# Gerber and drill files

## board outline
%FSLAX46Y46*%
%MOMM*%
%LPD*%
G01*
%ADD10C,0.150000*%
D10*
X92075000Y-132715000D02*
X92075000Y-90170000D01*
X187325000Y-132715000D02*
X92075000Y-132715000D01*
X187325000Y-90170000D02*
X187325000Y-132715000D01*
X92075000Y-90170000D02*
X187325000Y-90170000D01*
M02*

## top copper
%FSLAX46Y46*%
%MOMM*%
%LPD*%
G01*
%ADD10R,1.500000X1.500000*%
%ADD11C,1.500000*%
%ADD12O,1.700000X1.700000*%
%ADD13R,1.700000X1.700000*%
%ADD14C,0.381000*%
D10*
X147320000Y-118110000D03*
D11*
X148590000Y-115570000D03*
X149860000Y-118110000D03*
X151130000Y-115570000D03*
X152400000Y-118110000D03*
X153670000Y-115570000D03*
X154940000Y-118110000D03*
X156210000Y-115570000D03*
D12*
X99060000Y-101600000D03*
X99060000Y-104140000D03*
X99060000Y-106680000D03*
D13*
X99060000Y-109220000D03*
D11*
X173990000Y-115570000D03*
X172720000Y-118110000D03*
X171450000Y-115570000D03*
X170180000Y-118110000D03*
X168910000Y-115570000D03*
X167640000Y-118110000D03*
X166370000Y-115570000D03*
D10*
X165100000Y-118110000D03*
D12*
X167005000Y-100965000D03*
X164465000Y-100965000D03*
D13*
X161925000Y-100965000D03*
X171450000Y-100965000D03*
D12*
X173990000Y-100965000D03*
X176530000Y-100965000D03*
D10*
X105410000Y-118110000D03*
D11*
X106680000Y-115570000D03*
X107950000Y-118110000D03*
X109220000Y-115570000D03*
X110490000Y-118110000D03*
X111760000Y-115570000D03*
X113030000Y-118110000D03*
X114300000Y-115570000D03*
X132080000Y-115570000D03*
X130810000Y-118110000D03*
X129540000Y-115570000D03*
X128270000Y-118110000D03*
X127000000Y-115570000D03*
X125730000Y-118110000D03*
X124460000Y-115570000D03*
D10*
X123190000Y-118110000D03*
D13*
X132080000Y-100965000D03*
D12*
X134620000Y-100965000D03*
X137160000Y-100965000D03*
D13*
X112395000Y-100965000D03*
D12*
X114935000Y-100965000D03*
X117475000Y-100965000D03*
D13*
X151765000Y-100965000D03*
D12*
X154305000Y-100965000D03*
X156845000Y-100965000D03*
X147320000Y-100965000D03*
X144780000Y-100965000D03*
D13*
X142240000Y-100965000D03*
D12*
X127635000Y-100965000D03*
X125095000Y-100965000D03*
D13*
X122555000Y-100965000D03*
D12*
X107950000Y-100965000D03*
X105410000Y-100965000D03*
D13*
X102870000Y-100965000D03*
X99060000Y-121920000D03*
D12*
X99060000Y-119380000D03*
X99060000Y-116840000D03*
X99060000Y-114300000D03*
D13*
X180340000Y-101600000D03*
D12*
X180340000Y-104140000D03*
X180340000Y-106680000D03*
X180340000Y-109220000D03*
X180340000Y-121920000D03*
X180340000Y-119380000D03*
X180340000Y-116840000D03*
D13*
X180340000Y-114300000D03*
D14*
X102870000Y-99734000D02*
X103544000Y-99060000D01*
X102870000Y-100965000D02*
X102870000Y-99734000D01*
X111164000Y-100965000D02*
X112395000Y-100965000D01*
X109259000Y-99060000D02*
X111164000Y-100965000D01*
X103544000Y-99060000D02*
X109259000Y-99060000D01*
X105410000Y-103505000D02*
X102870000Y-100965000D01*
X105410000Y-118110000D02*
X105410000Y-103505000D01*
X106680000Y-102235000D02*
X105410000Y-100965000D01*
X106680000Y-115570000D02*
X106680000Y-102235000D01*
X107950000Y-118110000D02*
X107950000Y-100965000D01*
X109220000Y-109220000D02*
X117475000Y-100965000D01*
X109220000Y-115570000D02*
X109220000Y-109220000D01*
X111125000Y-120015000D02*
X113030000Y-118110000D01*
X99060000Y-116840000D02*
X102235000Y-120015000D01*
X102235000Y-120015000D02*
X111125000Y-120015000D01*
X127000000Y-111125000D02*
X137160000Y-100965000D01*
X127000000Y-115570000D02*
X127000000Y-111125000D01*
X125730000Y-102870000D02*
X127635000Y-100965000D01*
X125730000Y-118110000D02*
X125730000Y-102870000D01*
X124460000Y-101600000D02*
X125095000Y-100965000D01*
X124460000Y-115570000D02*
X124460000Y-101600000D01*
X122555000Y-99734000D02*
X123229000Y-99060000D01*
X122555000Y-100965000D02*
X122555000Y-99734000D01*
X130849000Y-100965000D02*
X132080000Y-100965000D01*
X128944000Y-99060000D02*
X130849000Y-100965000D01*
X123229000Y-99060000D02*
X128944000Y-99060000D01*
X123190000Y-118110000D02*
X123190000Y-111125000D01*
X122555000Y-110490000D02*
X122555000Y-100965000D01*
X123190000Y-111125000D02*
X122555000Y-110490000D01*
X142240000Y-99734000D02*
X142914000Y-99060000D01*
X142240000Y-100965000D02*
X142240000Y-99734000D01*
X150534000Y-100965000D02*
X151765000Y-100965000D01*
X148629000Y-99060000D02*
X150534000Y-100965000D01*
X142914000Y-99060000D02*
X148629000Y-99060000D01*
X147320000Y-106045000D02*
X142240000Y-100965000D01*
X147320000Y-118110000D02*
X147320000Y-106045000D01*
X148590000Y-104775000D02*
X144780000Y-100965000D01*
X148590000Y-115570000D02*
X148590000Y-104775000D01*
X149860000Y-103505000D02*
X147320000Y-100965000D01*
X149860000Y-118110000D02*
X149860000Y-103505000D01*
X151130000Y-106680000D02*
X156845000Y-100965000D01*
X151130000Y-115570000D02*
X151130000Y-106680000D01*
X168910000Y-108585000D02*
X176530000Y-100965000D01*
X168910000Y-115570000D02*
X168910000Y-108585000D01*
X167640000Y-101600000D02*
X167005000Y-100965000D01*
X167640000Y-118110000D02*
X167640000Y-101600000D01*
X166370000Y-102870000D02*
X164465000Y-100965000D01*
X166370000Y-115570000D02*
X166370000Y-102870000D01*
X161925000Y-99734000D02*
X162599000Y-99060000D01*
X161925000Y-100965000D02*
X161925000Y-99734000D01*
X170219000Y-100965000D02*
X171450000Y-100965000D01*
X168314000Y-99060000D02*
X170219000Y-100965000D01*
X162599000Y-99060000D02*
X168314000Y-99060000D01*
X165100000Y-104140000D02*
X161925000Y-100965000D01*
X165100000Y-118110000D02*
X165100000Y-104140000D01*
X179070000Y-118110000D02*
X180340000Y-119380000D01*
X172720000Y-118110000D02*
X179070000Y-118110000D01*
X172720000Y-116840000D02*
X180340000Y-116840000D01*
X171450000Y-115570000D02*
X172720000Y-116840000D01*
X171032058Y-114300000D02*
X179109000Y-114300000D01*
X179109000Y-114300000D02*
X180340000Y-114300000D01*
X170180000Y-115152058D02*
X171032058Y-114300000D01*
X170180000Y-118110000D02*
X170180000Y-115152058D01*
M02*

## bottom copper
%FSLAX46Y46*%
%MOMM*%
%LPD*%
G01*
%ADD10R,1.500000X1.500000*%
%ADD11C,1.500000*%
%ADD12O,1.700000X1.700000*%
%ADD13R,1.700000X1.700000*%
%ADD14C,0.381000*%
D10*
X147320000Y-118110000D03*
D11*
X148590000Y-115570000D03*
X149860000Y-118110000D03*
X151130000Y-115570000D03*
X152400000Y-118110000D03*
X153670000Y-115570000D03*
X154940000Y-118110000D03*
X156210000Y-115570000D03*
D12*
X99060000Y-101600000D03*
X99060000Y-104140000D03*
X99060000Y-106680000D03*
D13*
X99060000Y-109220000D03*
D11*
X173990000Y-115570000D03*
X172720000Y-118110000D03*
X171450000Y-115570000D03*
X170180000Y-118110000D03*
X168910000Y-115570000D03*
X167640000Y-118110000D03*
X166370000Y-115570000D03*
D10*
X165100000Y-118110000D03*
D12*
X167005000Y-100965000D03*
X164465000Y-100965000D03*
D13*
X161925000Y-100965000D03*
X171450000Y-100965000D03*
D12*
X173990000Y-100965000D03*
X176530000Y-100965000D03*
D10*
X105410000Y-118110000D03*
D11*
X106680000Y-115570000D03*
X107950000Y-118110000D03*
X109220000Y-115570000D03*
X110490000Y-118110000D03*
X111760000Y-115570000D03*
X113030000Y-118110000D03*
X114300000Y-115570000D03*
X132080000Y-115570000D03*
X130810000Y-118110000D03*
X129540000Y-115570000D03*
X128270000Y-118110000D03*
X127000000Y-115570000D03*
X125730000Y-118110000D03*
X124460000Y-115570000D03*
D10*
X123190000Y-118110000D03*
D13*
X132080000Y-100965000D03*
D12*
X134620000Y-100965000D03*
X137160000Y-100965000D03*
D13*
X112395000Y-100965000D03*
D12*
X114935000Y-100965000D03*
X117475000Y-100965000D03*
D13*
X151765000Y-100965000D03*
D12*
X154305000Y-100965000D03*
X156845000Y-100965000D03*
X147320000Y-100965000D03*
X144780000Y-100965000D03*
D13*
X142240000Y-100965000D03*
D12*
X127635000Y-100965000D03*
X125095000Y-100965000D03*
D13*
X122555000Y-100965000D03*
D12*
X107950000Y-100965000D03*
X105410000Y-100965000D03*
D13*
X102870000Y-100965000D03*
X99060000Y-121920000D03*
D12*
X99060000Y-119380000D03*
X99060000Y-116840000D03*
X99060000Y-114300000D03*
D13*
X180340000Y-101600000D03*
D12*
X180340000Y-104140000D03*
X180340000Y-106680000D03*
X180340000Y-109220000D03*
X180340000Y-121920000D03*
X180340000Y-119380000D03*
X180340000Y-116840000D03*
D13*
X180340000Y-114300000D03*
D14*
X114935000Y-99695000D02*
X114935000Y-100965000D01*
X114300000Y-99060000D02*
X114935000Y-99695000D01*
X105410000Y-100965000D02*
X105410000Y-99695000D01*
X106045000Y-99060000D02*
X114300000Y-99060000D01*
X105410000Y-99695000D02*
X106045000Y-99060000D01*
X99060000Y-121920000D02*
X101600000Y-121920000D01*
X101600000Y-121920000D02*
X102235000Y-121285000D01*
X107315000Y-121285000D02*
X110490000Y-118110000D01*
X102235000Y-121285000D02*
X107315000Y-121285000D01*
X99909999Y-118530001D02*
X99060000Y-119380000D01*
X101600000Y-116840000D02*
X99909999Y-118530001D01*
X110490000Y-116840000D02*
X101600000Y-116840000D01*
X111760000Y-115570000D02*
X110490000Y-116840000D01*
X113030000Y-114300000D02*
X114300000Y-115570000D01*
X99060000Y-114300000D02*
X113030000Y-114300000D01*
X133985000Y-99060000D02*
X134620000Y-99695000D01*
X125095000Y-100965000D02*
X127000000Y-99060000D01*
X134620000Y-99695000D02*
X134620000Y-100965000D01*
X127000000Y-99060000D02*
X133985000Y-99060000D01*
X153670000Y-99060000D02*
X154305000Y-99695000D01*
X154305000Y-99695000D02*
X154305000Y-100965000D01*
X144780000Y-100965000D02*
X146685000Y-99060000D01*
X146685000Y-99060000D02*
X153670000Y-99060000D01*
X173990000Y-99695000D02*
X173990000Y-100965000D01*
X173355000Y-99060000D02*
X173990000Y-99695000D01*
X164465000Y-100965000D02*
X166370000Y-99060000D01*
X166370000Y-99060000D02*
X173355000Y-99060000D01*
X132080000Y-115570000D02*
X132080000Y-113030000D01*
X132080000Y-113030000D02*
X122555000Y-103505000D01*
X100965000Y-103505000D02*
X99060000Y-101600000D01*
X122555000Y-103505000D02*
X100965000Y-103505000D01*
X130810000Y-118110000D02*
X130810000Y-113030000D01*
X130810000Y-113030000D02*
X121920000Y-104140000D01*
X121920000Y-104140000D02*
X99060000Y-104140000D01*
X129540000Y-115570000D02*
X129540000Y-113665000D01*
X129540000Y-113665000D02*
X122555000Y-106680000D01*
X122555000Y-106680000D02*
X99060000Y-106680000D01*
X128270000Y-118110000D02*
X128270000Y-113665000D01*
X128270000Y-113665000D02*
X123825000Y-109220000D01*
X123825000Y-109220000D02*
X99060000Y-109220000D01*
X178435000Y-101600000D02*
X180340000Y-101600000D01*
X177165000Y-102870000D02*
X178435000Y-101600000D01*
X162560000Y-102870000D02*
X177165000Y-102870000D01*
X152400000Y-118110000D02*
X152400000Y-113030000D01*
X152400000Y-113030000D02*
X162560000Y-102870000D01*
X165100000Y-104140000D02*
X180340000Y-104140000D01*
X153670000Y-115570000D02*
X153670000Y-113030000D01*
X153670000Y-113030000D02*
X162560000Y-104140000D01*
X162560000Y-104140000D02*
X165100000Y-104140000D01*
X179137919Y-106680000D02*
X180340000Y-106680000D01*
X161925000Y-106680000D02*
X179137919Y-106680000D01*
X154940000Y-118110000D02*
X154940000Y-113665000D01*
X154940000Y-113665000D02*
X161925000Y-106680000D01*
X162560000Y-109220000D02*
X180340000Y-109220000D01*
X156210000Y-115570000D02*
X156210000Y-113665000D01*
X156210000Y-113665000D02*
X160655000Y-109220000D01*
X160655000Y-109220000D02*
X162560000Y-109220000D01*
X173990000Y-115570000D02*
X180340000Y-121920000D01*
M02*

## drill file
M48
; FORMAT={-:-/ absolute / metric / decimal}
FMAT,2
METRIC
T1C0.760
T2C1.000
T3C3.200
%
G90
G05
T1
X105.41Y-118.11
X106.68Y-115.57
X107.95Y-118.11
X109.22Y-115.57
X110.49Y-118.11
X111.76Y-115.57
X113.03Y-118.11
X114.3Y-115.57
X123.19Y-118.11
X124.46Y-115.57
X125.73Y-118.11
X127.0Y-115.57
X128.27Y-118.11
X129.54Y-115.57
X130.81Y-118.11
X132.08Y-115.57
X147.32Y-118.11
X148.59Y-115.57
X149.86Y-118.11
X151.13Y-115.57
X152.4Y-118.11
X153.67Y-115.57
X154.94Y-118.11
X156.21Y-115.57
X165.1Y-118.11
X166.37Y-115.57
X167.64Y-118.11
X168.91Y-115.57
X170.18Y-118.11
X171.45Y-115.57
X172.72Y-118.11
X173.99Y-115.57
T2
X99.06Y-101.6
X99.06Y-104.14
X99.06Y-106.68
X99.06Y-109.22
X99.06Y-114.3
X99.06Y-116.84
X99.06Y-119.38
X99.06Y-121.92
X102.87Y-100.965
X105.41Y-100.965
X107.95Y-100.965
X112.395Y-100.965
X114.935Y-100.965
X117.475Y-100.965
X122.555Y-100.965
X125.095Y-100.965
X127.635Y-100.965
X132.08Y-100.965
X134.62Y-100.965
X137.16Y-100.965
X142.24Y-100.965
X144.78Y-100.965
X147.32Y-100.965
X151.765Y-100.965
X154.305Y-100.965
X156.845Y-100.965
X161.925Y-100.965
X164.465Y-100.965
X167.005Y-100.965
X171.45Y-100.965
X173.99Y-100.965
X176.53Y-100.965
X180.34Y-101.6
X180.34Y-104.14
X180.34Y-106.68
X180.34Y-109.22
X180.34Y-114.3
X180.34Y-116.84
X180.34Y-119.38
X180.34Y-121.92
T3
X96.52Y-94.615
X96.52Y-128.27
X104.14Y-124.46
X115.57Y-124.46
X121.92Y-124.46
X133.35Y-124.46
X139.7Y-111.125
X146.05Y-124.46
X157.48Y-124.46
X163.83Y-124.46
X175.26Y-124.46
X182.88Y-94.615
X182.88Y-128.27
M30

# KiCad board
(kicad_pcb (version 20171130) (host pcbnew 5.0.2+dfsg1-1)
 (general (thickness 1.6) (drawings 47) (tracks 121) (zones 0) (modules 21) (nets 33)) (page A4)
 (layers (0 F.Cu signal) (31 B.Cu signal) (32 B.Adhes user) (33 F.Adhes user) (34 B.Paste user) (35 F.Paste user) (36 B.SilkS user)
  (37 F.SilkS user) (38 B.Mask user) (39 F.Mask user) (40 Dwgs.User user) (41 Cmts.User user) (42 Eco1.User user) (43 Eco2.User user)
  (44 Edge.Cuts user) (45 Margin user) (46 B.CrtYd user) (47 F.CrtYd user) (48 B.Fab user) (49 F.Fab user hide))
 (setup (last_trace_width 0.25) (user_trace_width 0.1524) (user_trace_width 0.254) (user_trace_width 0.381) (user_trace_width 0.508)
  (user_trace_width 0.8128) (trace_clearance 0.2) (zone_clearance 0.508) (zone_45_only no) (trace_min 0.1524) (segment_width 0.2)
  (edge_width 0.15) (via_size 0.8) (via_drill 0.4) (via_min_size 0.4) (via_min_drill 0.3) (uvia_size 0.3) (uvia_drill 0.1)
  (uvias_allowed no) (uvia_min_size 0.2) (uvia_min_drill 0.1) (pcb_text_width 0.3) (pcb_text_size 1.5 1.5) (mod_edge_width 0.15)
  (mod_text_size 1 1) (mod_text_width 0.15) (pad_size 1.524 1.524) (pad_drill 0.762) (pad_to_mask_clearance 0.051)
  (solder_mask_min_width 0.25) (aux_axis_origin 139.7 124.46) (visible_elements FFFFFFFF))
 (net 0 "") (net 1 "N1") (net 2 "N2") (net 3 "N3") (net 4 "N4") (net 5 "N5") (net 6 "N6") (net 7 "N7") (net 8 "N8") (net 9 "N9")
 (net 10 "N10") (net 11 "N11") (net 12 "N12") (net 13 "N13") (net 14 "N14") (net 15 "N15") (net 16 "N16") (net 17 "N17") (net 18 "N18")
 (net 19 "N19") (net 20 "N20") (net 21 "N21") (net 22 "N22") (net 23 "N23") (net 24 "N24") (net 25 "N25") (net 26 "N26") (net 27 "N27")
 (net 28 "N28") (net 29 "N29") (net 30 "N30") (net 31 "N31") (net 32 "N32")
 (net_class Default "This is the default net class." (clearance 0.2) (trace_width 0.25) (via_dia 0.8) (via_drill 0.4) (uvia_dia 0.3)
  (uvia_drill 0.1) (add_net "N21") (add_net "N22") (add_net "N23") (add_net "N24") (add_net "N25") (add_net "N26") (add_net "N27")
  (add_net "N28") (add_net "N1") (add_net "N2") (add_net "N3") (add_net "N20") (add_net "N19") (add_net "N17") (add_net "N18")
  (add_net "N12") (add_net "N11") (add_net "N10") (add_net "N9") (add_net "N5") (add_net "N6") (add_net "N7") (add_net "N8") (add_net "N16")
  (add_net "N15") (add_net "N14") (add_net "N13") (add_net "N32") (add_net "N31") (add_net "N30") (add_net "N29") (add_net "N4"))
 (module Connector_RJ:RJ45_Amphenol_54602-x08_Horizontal (layer F.Cu) (at 147.32 118.11)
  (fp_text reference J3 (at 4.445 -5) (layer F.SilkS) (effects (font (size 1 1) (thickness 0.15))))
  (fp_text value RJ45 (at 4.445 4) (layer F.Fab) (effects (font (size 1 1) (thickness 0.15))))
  (pad "" np_thru_hole circle (at 10.16 6.35) (size 3.2 3.2) (drill 3.2) (layers *.Cu *.Mask))
  (pad "" np_thru_hole circle (at -1.27 6.35) (size 3.2 3.2) (drill 3.2) (layers *.Cu *.Mask))
  (pad 1 thru_hole rect (at 0 0) (size 1.5 1.5) (drill 0.76) (layers *.Cu *.Mask) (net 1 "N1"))
  (pad 2 thru_hole circle (at 1.27 -2.54) (size 1.5 1.5) (drill 0.76) (layers *.Cu *.Mask) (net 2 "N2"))
  (pad 3 thru_hole circle (at 2.54 0) (size 1.5 1.5) (drill 0.76) (layers *.Cu *.Mask) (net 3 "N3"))
  (pad 4 thru_hole circle (at 3.81 -2.54) (size 1.5 1.5) (drill 0.76) (layers *.Cu *.Mask) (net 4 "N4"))
  (pad 5 thru_hole circle (at 5.08 0) (size 1.5 1.5) (drill 0.76) (layers *.Cu *.Mask) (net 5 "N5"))
  (pad 6 thru_hole circle (at 6.35 -2.54) (size 1.5 1.5) (drill 0.76) (layers *.Cu *.Mask) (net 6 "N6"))
  (pad 7 thru_hole circle (at 7.62 0) (size 1.5 1.5) (drill 0.76) (layers *.Cu *.Mask) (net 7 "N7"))
  (pad 8 thru_hole circle (at 8.89 -2.54) (size 1.5 1.5) (drill 0.76) (layers *.Cu *.Mask) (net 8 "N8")))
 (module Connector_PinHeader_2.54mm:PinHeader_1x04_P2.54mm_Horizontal (layer F.Cu) (at 99.06 109.22 180)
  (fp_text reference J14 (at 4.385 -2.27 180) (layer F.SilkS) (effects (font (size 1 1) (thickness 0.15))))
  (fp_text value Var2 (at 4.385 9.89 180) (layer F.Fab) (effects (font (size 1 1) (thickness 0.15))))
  (pad 4 thru_hole oval (at 0 7.62 180) (size 1.7 1.7) (drill 1) (layers *.Cu *.Mask) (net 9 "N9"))
  (pad 3 thru_hole oval (at 0 5.08 180) (size 1.7 1.7) (drill 1) (layers *.Cu *.Mask) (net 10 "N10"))
  (pad 2 thru_hole oval (at 0 2.54 180) (size 1.7 1.7) (drill 1) (layers *.Cu *.Mask) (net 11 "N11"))
  (pad 1 thru_hole rect (at 0 0 180) (size 1.7 1.7) (drill 1) (layers *.Cu *.Mask) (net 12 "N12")))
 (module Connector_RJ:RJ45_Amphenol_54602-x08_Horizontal (layer F.Cu) (at 165.1 118.11)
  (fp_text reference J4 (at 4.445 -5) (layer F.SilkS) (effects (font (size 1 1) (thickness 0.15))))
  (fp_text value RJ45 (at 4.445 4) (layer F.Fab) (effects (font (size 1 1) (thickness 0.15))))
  (pad 8 thru_hole circle (at 8.89 -2.54) (size 1.5 1.5) (drill 0.76) (layers *.Cu *.Mask) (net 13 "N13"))
  (pad 7 thru_hole circle (at 7.62 0) (size 1.5 1.5) (drill 0.76) (layers *.Cu *.Mask) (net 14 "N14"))
  (pad 6 thru_hole circle (at 6.35 -2.54) (size 1.5 1.5) (drill 0.76) (layers *.Cu *.Mask) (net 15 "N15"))
  (pad 5 thru_hole circle (at 5.08 0) (size 1.5 1.5) (drill 0.76) (layers *.Cu *.Mask) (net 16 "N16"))
  (pad 4 thru_hole circle (at 3.81 -2.54) (size 1.5 1.5) (drill 0.76) (layers *.Cu *.Mask) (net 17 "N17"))
  (pad 3 thru_hole circle (at 2.54 0) (size 1.5 1.5) (drill 0.76) (layers *.Cu *.Mask) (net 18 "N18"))
  (pad 2 thru_hole circle (at 1.27 -2.54) (size 1.5 1.5) (drill 0.76) (layers *.Cu *.Mask) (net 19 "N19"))
  (pad 1 thru_hole rect (at 0 0) (size 1.5 1.5) (drill 0.76) (layers *.Cu *.Mask) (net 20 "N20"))
  (pad "" np_thru_hole circle (at -1.27 6.35) (size 3.2 3.2) (drill 3.2) (layers *.Cu *.Mask))
  (pad "" np_thru_hole circle (at 10.16 6.35) (size 3.2 3.2) (drill 3.2) (layers *.Cu *.Mask)))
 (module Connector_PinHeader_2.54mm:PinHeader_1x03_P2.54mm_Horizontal (layer F.Cu) (at 161.925 100.965 90)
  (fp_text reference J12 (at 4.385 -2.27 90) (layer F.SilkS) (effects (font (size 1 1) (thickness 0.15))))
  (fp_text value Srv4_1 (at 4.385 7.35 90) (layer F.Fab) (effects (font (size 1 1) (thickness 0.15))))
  (pad 3 thru_hole oval (at 0 5.08 90) (size 1.7 1.7) (drill 1) (layers *.Cu *.Mask) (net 18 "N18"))
  (pad 2 thru_hole oval (at 0 2.54 90) (size 1.7 1.7) (drill 1) (layers *.Cu *.Mask) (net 19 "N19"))
  (pad 1 thru_hole rect (at 0 0 90) (size 1.7 1.7) (drill 1) (layers *.Cu *.Mask) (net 20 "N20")))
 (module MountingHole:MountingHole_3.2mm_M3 (layer F.Cu) (at 139.7 111.125)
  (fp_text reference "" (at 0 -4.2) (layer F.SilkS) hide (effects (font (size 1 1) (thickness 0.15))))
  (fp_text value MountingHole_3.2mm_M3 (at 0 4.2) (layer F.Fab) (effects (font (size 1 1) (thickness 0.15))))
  (pad 1 np_thru_hole circle (at 0 0) (size 3.2 3.2) (drill 3.2) (layers *.Cu *.Mask)))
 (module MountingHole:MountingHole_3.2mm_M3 (layer F.Cu) (at 182.88 128.27)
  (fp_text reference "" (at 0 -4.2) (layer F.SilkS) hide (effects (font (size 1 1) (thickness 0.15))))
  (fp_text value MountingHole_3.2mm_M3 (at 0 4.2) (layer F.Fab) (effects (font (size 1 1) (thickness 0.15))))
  (pad 1 np_thru_hole circle (at 0 0) (size 3.2 3.2) (drill 3.2) (layers *.Cu *.Mask)))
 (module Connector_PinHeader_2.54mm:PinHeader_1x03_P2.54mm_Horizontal (layer F.Cu) (at 171.45 100.965 90)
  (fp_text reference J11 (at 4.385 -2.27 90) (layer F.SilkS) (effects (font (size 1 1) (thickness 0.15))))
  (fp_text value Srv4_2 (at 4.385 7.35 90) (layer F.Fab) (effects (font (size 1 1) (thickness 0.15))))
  (pad 1 thru_hole rect (at 0 0 90) (size 1.7 1.7) (drill 1) (layers *.Cu *.Mask) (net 20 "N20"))
  (pad 2 thru_hole oval (at 0 2.54 90) (size 1.7 1.7) (drill 1) (layers *.Cu *.Mask) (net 19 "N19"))
  (pad 3 thru_hole oval (at 0 5.08 90) (size 1.7 1.7) (drill 1) (layers *.Cu *.Mask) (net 17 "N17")))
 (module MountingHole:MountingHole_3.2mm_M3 (layer F.Cu) (at 96.52 128.27)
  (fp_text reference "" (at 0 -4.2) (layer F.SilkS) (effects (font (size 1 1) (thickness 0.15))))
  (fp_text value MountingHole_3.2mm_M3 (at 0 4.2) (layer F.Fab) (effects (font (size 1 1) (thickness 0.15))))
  (pad 1 np_thru_hole circle (at 0 0) (size 3.2 3.2) (drill 3.2) (layers *.Cu *.Mask)))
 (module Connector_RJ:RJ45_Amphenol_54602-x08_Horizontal (layer F.Cu) (at 105.41 118.11)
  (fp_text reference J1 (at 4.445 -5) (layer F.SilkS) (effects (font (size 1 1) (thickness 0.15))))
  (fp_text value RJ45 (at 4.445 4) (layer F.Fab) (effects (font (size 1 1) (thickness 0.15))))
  (pad "" np_thru_hole circle (at 10.16 6.35) (size 3.2 3.2) (drill 3.2) (layers *.Cu *.Mask))
  (pad "" np_thru_hole circle (at -1.27 6.35) (size 3.2 3.2) (drill 3.2) (layers *.Cu *.Mask))
  (pad 1 thru_hole rect (at 0 0) (size 1.5 1.5) (drill 0.76) (layers *.Cu *.Mask) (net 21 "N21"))
  (pad 2 thru_hole circle (at 1.27 -2.54) (size 1.5 1.5) (drill 0.76) (layers *.Cu *.Mask) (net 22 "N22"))
  (pad 3 thru_hole circle (at 2.54 0) (size 1.5 1.5) (drill 0.76) (layers *.Cu *.Mask) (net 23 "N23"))
  (pad 4 thru_hole circle (at 3.81 -2.54) (size 1.5 1.5) (drill 0.76) (layers *.Cu *.Mask) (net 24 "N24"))
  (pad 5 thru_hole circle (at 5.08 0) (size 1.5 1.5) (drill 0.76) (layers *.Cu *.Mask) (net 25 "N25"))
  (pad 6 thru_hole circle (at 6.35 -2.54) (size 1.5 1.5) (drill 0.76) (layers *.Cu *.Mask) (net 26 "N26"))
  (pad 7 thru_hole circle (at 7.62 0) (size 1.5 1.5) (drill 0.76) (layers *.Cu *.Mask) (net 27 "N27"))
  (pad 8 thru_hole circle (at 8.89 -2.54) (size 1.5 1.5) (drill 0.76) (layers *.Cu *.Mask) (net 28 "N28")))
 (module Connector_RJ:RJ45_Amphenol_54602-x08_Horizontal (layer F.Cu) (at 123.19 118.11)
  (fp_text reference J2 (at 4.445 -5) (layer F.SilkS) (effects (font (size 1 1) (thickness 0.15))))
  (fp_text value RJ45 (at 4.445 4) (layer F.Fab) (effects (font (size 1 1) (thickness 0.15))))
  (pad 8 thru_hole circle (at 8.89 -2.54) (size 1.5 1.5) (drill 0.76) (layers *.Cu *.Mask) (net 9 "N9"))
  (pad 7 thru_hole circle (at 7.62 0) (size 1.5 1.5) (drill 0.76) (layers *.Cu *.Mask) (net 10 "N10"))
  (pad 6 thru_hole circle (at 6.35 -2.54) (size 1.5 1.5) (drill 0.76) (layers *.Cu *.Mask) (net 11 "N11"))
  (pad 5 thru_hole circle (at 5.08 0) (size 1.5 1.5) (drill 0.76) (layers *.Cu *.Mask) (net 12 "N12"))
  (pad 4 thru_hole circle (at 3.81 -2.54) (size 1.5 1.5) (drill 0.76) (layers *.Cu *.Mask) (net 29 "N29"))
  (pad 3 thru_hole circle (at 2.54 0) (size 1.5 1.5) (drill 0.76) (layers *.Cu *.Mask) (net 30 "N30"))
  (pad 2 thru_hole circle (at 1.27 -2.54) (size 1.5 1.5) (drill 0.76) (layers *.Cu *.Mask) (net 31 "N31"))
  (pad 1 thru_hole rect (at 0 0) (size 1.5 1.5) (drill 0.76) (layers *.Cu *.Mask) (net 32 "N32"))
  (pad "" np_thru_hole circle (at -1.27 6.35) (size 3.2 3.2) (drill 3.2) (layers *.Cu *.Mask))
  (pad "" np_thru_hole circle (at 10.16 6.35) (size 3.2 3.2) (drill 3.2) (layers *.Cu *.Mask)))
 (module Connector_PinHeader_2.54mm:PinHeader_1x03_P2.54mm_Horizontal (layer F.Cu) (at 132.08 100.965 90)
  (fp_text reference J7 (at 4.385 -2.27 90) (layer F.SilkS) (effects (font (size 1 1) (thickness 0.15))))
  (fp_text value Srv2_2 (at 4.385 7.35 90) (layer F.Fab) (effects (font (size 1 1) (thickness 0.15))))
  (pad 1 thru_hole rect (at 0 0 90) (size 1.7 1.7) (drill 1) (layers *.Cu *.Mask) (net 32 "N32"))
  (pad 2 thru_hole oval (at 0 2.54 90) (size 1.7 1.7) (drill 1) (layers *.Cu *.Mask) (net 31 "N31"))
  (pad 3 thru_hole oval (at 0 5.08 90) (size 1.7 1.7) (drill 1) (layers *.Cu *.Mask) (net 29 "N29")))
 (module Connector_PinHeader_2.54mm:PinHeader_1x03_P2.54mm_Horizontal (layer F.Cu) (at 112.395 100.965 90)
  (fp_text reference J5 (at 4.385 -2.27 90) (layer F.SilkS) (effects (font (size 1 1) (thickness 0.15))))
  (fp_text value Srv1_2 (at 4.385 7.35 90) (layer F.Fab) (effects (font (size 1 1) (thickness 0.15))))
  (pad 1 thru_hole rect (at 0 0 90) (size 1.7 1.7) (drill 1) (layers *.Cu *.Mask) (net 21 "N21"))
  (pad 2 thru_hole oval (at 0 2.54 90) (size 1.7 1.7) (drill 1) (layers *.Cu *.Mask) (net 22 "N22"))
  (pad 3 thru_hole oval (at 0 5.08 90) (size 1.7 1.7) (drill 1) (layers *.Cu *.Mask) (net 24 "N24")))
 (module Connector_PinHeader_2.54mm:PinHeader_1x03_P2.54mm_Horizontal (layer F.Cu) (at 151.765 100.965 90)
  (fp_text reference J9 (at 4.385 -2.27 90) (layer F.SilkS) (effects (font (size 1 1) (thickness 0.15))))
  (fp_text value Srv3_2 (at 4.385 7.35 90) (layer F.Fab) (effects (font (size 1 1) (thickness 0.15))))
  (pad 1 thru_hole rect (at 0 0 90) (size 1.7 1.7) (drill 1) (layers *.Cu *.Mask) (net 1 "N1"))
  (pad 2 thru_hole oval (at 0 2.54 90) (size 1.7 1.7) (drill 1) (layers *.Cu *.Mask) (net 2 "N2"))
  (pad 3 thru_hole oval (at 0 5.08 90) (size 1.7 1.7) (drill 1) (layers *.Cu *.Mask) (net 4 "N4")))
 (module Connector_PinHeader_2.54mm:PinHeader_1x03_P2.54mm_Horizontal (layer F.Cu) (at 142.24 100.965 90)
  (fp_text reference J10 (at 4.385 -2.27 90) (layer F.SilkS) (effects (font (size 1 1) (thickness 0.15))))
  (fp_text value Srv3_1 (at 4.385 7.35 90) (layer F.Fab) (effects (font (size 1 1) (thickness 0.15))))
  (pad 3 thru_hole oval (at 0 5.08 90) (size 1.7 1.7) (drill 1) (layers *.Cu *.Mask) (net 3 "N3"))
  (pad 2 thru_hole oval (at 0 2.54 90) (size 1.7 1.7) (drill 1) (layers *.Cu *.Mask) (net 2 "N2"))
  (pad 1 thru_hole rect (at 0 0 90) (size 1.7 1.7) (drill 1) (layers *.Cu *.Mask) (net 1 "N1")))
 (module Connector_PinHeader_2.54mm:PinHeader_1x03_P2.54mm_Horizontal (layer F.Cu) (at 122.555 100.965 90)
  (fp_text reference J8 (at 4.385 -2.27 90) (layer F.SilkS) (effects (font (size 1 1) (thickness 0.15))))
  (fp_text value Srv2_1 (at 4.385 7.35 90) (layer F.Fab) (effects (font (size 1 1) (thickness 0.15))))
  (pad 3 thru_hole oval (at 0 5.08 90) (size 1.7 1.7) (drill 1) (layers *.Cu *.Mask) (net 30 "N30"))
  (pad 2 thru_hole oval (at 0 2.54 90) (size 1.7 1.7) (drill 1) (layers *.Cu *.Mask) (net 31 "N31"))
  (pad 1 thru_hole rect (at 0 0 90) (size 1.7 1.7) (drill 1) (layers *.Cu *.Mask) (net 32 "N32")))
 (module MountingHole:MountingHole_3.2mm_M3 (layer F.Cu) (at 182.88 94.615)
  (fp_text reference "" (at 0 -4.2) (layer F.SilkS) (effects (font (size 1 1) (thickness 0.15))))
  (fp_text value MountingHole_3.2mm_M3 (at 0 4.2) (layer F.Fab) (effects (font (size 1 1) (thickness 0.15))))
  (pad 1 np_thru_hole circle (at 0 0) (size 3.2 3.2) (drill 3.2) (layers *.Cu *.Mask)))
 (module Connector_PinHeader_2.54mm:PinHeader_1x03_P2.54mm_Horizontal (layer F.Cu) (at 102.87 100.965 90)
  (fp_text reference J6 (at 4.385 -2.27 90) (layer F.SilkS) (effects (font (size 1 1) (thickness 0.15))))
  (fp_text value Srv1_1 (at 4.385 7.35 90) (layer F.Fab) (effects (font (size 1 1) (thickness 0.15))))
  (pad 3 thru_hole oval (at 0 5.08 90) (size 1.7 1.7) (drill 1) (layers *.Cu *.Mask) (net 23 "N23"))
  (pad 2 thru_hole oval (at 0 2.54 90) (size 1.7 1.7) (drill 1) (layers *.Cu *.Mask) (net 22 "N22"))
  (pad 1 thru_hole rect (at 0 0 90) (size 1.7 1.7) (drill 1) (layers *.Cu *.Mask) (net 21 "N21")))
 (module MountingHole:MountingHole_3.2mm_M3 (layer F.Cu) (at 96.52 94.615)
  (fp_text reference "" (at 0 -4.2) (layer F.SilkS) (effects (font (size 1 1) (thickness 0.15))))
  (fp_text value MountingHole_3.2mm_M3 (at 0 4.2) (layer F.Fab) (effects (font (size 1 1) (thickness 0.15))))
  (pad 1 np_thru_hole circle (at 0 0) (size 3.2 3.2) (drill 3.2) (layers *.Cu *.Mask)))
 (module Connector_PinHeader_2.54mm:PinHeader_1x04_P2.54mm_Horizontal (layer F.Cu) (at 99.06 121.92 180)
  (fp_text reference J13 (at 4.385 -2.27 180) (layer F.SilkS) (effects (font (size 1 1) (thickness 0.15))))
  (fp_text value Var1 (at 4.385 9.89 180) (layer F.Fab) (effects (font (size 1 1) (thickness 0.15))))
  (pad 1 thru_hole rect (at 0 0 180) (size 1.7 1.7) (drill 1) (layers *.Cu *.Mask) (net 25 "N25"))
  (pad 2 thru_hole oval (at 0 2.54 180) (size 1.7 1.7) (drill 1) (layers *.Cu *.Mask) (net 26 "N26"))
  (pad 3 thru_hole oval (at 0 5.08 180) (size 1.7 1.7) (drill 1) (layers *.Cu *.Mask) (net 27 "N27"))
  (pad 4 thru_hole oval (at 0 7.62 180) (size 1.7 1.7) (drill 1) (layers *.Cu *.Mask) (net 28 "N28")))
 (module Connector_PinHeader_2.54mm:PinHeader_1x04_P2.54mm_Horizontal (layer F.Cu) (at 180.34 101.6)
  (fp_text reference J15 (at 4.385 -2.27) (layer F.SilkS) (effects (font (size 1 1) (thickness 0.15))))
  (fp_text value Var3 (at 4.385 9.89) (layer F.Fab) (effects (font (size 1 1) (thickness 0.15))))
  (pad 1 thru_hole rect (at 0 0) (size 1.7 1.7) (drill 1) (layers *.Cu *.Mask) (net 5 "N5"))
  (pad 2 thru_hole oval (at 0 2.54) (size 1.7 1.7) (drill 1) (layers *.Cu *.Mask) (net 6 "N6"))
  (pad 3 thru_hole oval (at 0 5.08) (size 1.7 1.7) (drill 1) (layers *.Cu *.Mask) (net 7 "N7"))
  (pad 4 thru_hole oval (at 0 7.62) (size 1.7 1.7) (drill 1) (layers *.Cu *.Mask) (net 8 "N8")))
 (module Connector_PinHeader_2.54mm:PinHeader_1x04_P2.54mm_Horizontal (layer F.Cu) (at 180.34 114.3)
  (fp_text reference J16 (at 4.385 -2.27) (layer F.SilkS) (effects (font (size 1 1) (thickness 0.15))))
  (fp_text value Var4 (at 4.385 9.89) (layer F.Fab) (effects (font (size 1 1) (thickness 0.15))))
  (pad 4 thru_hole oval (at 0 7.62) (size 1.7 1.7) (drill 1) (layers *.Cu *.Mask) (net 13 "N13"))
  (pad 3 thru_hole oval (at 0 5.08) (size 1.7 1.7) (drill 1) (layers *.Cu *.Mask) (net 14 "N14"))
  (pad 2 thru_hole oval (at 0 2.54) (size 1.7 1.7) (drill 1) (layers *.Cu *.Mask) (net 15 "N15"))
  (pad 1 thru_hole rect (at 0 0) (size 1.7 1.7) (drill 1) (layers *.Cu *.Mask) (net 16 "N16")))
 (gr_line (start 92.075 132.715) (end 92.075 90.17) (layer Edge.Cuts) (width 0.15))
 (gr_line (start 187.325 132.715) (end 92.075 132.715) (layer Edge.Cuts) (width 0.15))
 (gr_line (start 187.325 90.17) (end 187.325 132.715) (layer Edge.Cuts) (width 0.15))
 (gr_line (start 92.075 90.17) (end 187.325 90.17) (layer Edge.Cuts) (width 0.15))
 (segment (start 102.87 99.734) (end 103.544 99.06) (width 0.381) (layer F.Cu) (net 21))
 (segment (start 102.87 100.965) (end 102.87 99.734) (width 0.381) (layer F.Cu) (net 21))
 (segment (start 111.164 100.965) (end 112.395 100.965) (width 0.381) (layer F.Cu) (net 21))
 (segment (start 109.259 99.06) (end 111.164 100.965) (width 0.381) (layer F.Cu) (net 21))
 (segment (start 103.544 99.06) (end 109.259 99.06) (width 0.381) (layer F.Cu) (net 21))
 (segment (start 105.41 103.505) (end 102.87 100.965) (width 0.381) (layer F.Cu) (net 21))
 (segment (start 105.41 118.11) (end 105.41 103.505) (width 0.381) (layer F.Cu) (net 21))
 (segment (start 106.68 102.235) (end 105.41 100.965) (width 0.381) (layer F.Cu) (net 22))
 (segment (start 106.68 115.57) (end 106.68 102.235) (width 0.381) (layer F.Cu) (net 22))
 (segment (start 114.935 99.695) (end 114.935 100.965) (width 0.381) (layer B.Cu) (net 22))
 (segment (start 114.3 99.06) (end 114.935 99.695) (width 0.381) (layer B.Cu) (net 22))
 (segment (start 105.41 100.965) (end 105.41 99.695) (width 0.381) (layer B.Cu) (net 22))
 (segment (start 106.045 99.06) (end 114.3 99.06) (width 0.381) (layer B.Cu) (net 22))
 (segment (start 105.41 99.695) (end 106.045 99.06) (width 0.381) (layer B.Cu) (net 22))
 (segment (start 107.95 118.11) (end 107.95 100.965) (width 0.381) (layer F.Cu) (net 23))
 (segment (start 109.22 109.22) (end 117.475 100.965) (width 0.381) (layer F.Cu) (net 24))
 (segment (start 109.22 115.57) (end 109.22 109.22) (width 0.381) (layer F.Cu) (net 24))
 (segment (start 99.06 121.92) (end 101.6 121.92) (width 0.381) (layer B.Cu) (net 25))
 (segment (start 101.6 121.92) (end 102.235 121.285) (width 0.381) (layer B.Cu) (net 25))
 (segment (start 107.315 121.285) (end 110.49 118.11) (width 0.381) (layer B.Cu) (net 25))
 (segment (start 102.235 121.285) (end 107.315 121.285) (width 0.381) (layer B.Cu) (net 25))
 (segment (start 99.909999 118.530001) (end 99.06 119.38) (width 0.381) (layer B.Cu) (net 26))
 (segment (start 101.6 116.84) (end 99.909999 118.530001) (width 0.381) (layer B.Cu) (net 26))
 (segment (start 110.49 116.84) (end 101.6 116.84) (width 0.381) (layer B.Cu) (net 26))
 (segment (start 111.76 115.57) (end 110.49 116.84) (width 0.381) (layer B.Cu) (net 26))
 (segment (start 111.125 120.015) (end 113.03 118.11) (width 0.381) (layer F.Cu) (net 27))
 (segment (start 99.06 116.84) (end 102.235 120.015) (width 0.381) (layer F.Cu) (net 27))
 (segment (start 102.235 120.015) (end 111.125 120.015) (width 0.381) (layer F.Cu) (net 27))
 (segment (start 113.03 114.3) (end 114.3 115.57) (width 0.381) (layer B.Cu) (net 28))
 (segment (start 99.06 114.3) (end 113.03 114.3) (width 0.381) (layer B.Cu) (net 28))
 (segment (start 127 111.125) (end 137.16 100.965) (width 0.381) (layer F.Cu) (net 29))
 (segment (start 127 115.57) (end 127 111.125) (width 0.381) (layer F.Cu) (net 29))
 (segment (start 125.73 102.87) (end 127.635 100.965) (width 0.381) (layer F.Cu) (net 30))
 (segment (start 125.73 118.11) (end 125.73 102.87) (width 0.381) (layer F.Cu) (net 30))
 (segment (start 124.46 101.6) (end 125.095 100.965) (width 0.381) (layer F.Cu) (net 31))
 (segment (start 124.46 115.57) (end 124.46 101.6) (width 0.381) (layer F.Cu) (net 31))
 (segment (start 133.985 99.06) (end 134.62 99.695) (width 0.381) (layer B.Cu) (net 31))
 (segment (start 125.095 100.965) (end 127 99.06) (width 0.381) (layer B.Cu) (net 31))
 (segment (start 134.62 99.695) (end 134.62 100.965) (width 0.381) (layer B.Cu) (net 31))
 (segment (start 127 99.06) (end 133.985 99.06) (width 0.381) (layer B.Cu) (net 31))
 (segment (start 122.555 99.734) (end 123.229 99.06) (width 0.381) (layer F.Cu) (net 32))
 (segment (start 122.555 100.965) (end 122.555 99.734) (width 0.381) (layer F.Cu) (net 32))
 (segment (start 130.849 100.965) (end 132.08 100.965) (width 0.381) (layer F.Cu) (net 32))
 (segment (start 128.944 99.06) (end 130.849 100.965) (width 0.381) (layer F.Cu) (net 32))
 (segment (start 123.229 99.06) (end 128.944 99.06) (width 0.381) (layer F.Cu) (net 32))
 (segment (start 123.19 118.11) (end 123.19 111.125) (width 0.381) (layer F.Cu) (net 32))
 (segment (start 122.555 110.49) (end 122.555 100.965) (width 0.381) (layer F.Cu) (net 32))
 (segment (start 123.19 111.125) (end 122.555 110.49) (width 0.381) (layer F.Cu) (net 32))
 (segment (start 142.24 99.734) (end 142.914 99.06) (width 0.381) (layer F.Cu) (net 1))
 (segment (start 142.24 100.965) (end 142.24 99.734) (width 0.381) (layer F.Cu) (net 1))
 (segment (start 150.534 100.965) (end 151.765 100.965) (width 0.381) (layer F.Cu) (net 1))
 (segment (start 148.629 99.06) (end 150.534 100.965) (width 0.381) (layer F.Cu) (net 1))
 (segment (start 142.914 99.06) (end 148.629 99.06) (width 0.381) (layer F.Cu) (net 1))
 (segment (start 147.32 106.045) (end 142.24 100.965) (width 0.381) (layer F.Cu) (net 1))
 (segment (start 147.32 118.11) (end 147.32 106.045) (width 0.381) (layer F.Cu) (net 1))
 (segment (start 148.59 104.775) (end 144.78 100.965) (width 0.381) (layer F.Cu) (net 2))
 (segment (start 148.59 115.57) (end 148.59 104.775) (width 0.381) (layer F.Cu) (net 2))
 (segment (start 153.67 99.06) (end 154.305 99.695) (width 0.381) (layer B.Cu) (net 2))
 (segment (start 154.305 99.695) (end 154.305 100.965) (width 0.381) (layer B.Cu) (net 2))
 (segment (start 144.78 100.965) (end 146.685 99.06) (width 0.381) (layer B.Cu) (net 2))
 (segment (start 146.685 99.06) (end 153.67 99.06) (width 0.381) (layer B.Cu) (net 2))
 (segment (start 149.86 103.505) (end 147.32 100.965) (width 0.381) (layer F.Cu) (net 3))
 (segment (start 149.86 118.11) (end 149.86 103.505) (width 0.381) (layer F.Cu) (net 3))
 (segment (start 151.13 106.68) (end 156.845 100.965) (width 0.381) (layer F.Cu) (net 4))
 (segment (start 151.13 115.57) (end 151.13 106.68) (width 0.381) (layer F.Cu) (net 4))
 (segment (start 168.91 108.585) (end 176.53 100.965) (width 0.381) (layer F.Cu) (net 17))
 (segment (start 168.91 115.57) (end 168.91 108.585) (width 0.381) (layer F.Cu) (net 17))
 (segment (start 167.64 101.6) (end 167.005 100.965) (width 0.381) (layer F.Cu) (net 18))
 (segment (start 167.64 118.11) (end 167.64 101.6) (width 0.381) (layer F.Cu) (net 18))
 (segment (start 166.37 102.87) (end 164.465 100.965) (width 0.381) (layer F.Cu) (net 19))
 (segment (start 166.37 115.57) (end 166.37 102.87) (width 0.381) (layer F.Cu) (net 19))
 (segment (start 173.99 99.695) (end 173.99 100.965) (width 0.381) (layer B.Cu) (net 19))
 (segment (start 173.355 99.06) (end 173.99 99.695) (width 0.381) (layer B.Cu) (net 19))
 (segment (start 164.465 100.965) (end 166.37 99.06) (width 0.381) (layer B.Cu) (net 19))
 (segment (start 166.37 99.06) (end 173.355 99.06) (width 0.381) (layer B.Cu) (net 19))
 (segment (start 161.925 99.734) (end 162.599 99.06) (width 0.381) (layer F.Cu) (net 20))
 (segment (start 161.925 100.965) (end 161.925 99.734) (width 0.381) (layer F.Cu) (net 20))
 (segment (start 170.219 100.965) (end 171.45 100.965) (width 0.381) (layer F.Cu) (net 20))
 (segment (start 168.314 99.06) (end 170.219 100.965) (width 0.381) (layer F.Cu) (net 20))
 (segment (start 162.599 99.06) (end 168.314 99.06) (width 0.381) (layer F.Cu) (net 20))
 (segment (start 165.1 104.14) (end 161.925 100.965) (width 0.381) (layer F.Cu) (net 20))
 (segment (start 165.1 118.11) (end 165.1 104.14) (width 0.381) (layer F.Cu) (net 20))
 (segment (start 132.08 115.57) (end 132.08 113.03) (width 0.381) (layer B.Cu) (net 9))
 (segment (start 132.08 113.03) (end 122.555 103.505) (width 0.381) (layer B.Cu) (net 9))
 (segment (start 100.965 103.505) (end 99.06 101.6) (width 0.381) (layer B.Cu) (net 9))
 (segment (start 122.555 103.505) (end 100.965 103.505) (width 0.381) (layer B.Cu) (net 9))
 (segment (start 130.81 118.11) (end 130.81 113.03) (width 0.381) (layer B.Cu) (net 10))
 (segment (start 130.81 113.03) (end 121.92 104.14) (width 0.381) (layer B.Cu) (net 10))
 (segment (start 121.92 104.14) (end 99.06 104.14) (width 0.381) (layer B.Cu) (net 10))
 (segment (start 129.54 115.57) (end 129.54 113.665) (width 0.381) (layer B.Cu) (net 11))
 (segment (start 129.54 113.665) (end 122.555 106.68) (width 0.381) (layer B.Cu) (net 11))
 (segment (start 122.555 106.68) (end 99.06 106.68) (width 0.381) (layer B.Cu) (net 11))
 (segment (start 128.27 118.11) (end 128.27 113.665) (width 0.381) (layer B.Cu) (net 12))
 (segment (start 128.27 113.665) (end 123.825 109.22) (width 0.381) (layer B.Cu) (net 12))
 (segment (start 123.825 109.22) (end 99.06 109.22) (width 0.381) (layer B.Cu) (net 12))
 (segment (start 178.435 101.6) (end 180.34 101.6) (width 0.381) (layer B.Cu) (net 5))
 (segment (start 177.165 102.87) (end 178.435 101.6) (width 0.381) (layer B.Cu) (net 5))
 (segment (start 162.56 102.87) (end 177.165 102.87) (width 0.381) (layer B.Cu) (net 5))
 (segment (start 152.4 118.11) (end 152.4 113.03) (width 0.381) (layer B.Cu) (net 5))
 (segment (start 152.4 113.03) (end 162.56 102.87) (width 0.381) (layer B.Cu) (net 5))
 (segment (start 165.1 104.14) (end 180.34 104.14) (width 0.381) (layer B.Cu) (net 6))
 (segment (start 153.67 115.57) (end 153.67 113.03) (width 0.381) (layer B.Cu) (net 6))
 (segment (start 153.67 113.03) (end 162.56 104.14) (width 0.381) (layer B.Cu) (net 6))
 (segment (start 162.56 104.14) (end 165.1 104.14) (width 0.381) (layer B.Cu) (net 6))
 (segment (start 179.137919 106.68) (end 180.34 106.68) (width 0.381) (layer B.Cu) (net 7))
 (segment (start 161.925 106.68) (end 179.137919 106.68) (width 0.381) (layer B.Cu) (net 7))
 (segment (start 154.94 118.11) (end 154.94 113.665) (width 0.381) (layer B.Cu) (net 7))
 (segment (start 154.94 113.665) (end 161.925 106.68) (width 0.381) (layer B.Cu) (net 7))
 (segment (start 162.56 109.22) (end 180.34 109.22) (width 0.381) (layer B.Cu) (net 8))
 (segment (start 156.21 115.57) (end 156.21 113.665) (width 0.381) (layer B.Cu) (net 8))
 (segment (start 156.21 113.665) (end 160.655 109.22) (width 0.381) (layer B.Cu) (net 8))
 (segment (start 160.655 109.22) (end 162.56 109.22) (width 0.381) (layer B.Cu) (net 8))
 (segment (start 173.99 115.57) (end 180.34 121.92) (width 0.381) (layer B.Cu) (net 13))
 (segment (start 179.07 118.11) (end 180.34 119.38) (width 0.381) (layer F.Cu) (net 14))
 (segment (start 172.72 118.11) (end 179.07 118.11) (width 0.381) (layer F.Cu) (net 14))
 (segment (start 172.72 116.84) (end 180.34 116.84) (width 0.381) (layer F.Cu) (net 15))
 (segment (start 171.45 115.57) (end 172.72 116.84) (width 0.381) (layer F.Cu) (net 15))
 (segment (start 171.032058 114.3) (end 179.109 114.3) (width 0.381) (layer F.Cu) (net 16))
 (segment (start 179.109 114.3) (end 180.34 114.3) (width 0.381) (layer F.Cu) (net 16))
 (segment (start 170.18 115.152058) (end 171.032058 114.3) (width 0.381) (layer F.Cu) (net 16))
 (segment (start 170.18 118.11) (end 170.18 115.152058) (width 0.381) (layer F.Cu) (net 16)))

